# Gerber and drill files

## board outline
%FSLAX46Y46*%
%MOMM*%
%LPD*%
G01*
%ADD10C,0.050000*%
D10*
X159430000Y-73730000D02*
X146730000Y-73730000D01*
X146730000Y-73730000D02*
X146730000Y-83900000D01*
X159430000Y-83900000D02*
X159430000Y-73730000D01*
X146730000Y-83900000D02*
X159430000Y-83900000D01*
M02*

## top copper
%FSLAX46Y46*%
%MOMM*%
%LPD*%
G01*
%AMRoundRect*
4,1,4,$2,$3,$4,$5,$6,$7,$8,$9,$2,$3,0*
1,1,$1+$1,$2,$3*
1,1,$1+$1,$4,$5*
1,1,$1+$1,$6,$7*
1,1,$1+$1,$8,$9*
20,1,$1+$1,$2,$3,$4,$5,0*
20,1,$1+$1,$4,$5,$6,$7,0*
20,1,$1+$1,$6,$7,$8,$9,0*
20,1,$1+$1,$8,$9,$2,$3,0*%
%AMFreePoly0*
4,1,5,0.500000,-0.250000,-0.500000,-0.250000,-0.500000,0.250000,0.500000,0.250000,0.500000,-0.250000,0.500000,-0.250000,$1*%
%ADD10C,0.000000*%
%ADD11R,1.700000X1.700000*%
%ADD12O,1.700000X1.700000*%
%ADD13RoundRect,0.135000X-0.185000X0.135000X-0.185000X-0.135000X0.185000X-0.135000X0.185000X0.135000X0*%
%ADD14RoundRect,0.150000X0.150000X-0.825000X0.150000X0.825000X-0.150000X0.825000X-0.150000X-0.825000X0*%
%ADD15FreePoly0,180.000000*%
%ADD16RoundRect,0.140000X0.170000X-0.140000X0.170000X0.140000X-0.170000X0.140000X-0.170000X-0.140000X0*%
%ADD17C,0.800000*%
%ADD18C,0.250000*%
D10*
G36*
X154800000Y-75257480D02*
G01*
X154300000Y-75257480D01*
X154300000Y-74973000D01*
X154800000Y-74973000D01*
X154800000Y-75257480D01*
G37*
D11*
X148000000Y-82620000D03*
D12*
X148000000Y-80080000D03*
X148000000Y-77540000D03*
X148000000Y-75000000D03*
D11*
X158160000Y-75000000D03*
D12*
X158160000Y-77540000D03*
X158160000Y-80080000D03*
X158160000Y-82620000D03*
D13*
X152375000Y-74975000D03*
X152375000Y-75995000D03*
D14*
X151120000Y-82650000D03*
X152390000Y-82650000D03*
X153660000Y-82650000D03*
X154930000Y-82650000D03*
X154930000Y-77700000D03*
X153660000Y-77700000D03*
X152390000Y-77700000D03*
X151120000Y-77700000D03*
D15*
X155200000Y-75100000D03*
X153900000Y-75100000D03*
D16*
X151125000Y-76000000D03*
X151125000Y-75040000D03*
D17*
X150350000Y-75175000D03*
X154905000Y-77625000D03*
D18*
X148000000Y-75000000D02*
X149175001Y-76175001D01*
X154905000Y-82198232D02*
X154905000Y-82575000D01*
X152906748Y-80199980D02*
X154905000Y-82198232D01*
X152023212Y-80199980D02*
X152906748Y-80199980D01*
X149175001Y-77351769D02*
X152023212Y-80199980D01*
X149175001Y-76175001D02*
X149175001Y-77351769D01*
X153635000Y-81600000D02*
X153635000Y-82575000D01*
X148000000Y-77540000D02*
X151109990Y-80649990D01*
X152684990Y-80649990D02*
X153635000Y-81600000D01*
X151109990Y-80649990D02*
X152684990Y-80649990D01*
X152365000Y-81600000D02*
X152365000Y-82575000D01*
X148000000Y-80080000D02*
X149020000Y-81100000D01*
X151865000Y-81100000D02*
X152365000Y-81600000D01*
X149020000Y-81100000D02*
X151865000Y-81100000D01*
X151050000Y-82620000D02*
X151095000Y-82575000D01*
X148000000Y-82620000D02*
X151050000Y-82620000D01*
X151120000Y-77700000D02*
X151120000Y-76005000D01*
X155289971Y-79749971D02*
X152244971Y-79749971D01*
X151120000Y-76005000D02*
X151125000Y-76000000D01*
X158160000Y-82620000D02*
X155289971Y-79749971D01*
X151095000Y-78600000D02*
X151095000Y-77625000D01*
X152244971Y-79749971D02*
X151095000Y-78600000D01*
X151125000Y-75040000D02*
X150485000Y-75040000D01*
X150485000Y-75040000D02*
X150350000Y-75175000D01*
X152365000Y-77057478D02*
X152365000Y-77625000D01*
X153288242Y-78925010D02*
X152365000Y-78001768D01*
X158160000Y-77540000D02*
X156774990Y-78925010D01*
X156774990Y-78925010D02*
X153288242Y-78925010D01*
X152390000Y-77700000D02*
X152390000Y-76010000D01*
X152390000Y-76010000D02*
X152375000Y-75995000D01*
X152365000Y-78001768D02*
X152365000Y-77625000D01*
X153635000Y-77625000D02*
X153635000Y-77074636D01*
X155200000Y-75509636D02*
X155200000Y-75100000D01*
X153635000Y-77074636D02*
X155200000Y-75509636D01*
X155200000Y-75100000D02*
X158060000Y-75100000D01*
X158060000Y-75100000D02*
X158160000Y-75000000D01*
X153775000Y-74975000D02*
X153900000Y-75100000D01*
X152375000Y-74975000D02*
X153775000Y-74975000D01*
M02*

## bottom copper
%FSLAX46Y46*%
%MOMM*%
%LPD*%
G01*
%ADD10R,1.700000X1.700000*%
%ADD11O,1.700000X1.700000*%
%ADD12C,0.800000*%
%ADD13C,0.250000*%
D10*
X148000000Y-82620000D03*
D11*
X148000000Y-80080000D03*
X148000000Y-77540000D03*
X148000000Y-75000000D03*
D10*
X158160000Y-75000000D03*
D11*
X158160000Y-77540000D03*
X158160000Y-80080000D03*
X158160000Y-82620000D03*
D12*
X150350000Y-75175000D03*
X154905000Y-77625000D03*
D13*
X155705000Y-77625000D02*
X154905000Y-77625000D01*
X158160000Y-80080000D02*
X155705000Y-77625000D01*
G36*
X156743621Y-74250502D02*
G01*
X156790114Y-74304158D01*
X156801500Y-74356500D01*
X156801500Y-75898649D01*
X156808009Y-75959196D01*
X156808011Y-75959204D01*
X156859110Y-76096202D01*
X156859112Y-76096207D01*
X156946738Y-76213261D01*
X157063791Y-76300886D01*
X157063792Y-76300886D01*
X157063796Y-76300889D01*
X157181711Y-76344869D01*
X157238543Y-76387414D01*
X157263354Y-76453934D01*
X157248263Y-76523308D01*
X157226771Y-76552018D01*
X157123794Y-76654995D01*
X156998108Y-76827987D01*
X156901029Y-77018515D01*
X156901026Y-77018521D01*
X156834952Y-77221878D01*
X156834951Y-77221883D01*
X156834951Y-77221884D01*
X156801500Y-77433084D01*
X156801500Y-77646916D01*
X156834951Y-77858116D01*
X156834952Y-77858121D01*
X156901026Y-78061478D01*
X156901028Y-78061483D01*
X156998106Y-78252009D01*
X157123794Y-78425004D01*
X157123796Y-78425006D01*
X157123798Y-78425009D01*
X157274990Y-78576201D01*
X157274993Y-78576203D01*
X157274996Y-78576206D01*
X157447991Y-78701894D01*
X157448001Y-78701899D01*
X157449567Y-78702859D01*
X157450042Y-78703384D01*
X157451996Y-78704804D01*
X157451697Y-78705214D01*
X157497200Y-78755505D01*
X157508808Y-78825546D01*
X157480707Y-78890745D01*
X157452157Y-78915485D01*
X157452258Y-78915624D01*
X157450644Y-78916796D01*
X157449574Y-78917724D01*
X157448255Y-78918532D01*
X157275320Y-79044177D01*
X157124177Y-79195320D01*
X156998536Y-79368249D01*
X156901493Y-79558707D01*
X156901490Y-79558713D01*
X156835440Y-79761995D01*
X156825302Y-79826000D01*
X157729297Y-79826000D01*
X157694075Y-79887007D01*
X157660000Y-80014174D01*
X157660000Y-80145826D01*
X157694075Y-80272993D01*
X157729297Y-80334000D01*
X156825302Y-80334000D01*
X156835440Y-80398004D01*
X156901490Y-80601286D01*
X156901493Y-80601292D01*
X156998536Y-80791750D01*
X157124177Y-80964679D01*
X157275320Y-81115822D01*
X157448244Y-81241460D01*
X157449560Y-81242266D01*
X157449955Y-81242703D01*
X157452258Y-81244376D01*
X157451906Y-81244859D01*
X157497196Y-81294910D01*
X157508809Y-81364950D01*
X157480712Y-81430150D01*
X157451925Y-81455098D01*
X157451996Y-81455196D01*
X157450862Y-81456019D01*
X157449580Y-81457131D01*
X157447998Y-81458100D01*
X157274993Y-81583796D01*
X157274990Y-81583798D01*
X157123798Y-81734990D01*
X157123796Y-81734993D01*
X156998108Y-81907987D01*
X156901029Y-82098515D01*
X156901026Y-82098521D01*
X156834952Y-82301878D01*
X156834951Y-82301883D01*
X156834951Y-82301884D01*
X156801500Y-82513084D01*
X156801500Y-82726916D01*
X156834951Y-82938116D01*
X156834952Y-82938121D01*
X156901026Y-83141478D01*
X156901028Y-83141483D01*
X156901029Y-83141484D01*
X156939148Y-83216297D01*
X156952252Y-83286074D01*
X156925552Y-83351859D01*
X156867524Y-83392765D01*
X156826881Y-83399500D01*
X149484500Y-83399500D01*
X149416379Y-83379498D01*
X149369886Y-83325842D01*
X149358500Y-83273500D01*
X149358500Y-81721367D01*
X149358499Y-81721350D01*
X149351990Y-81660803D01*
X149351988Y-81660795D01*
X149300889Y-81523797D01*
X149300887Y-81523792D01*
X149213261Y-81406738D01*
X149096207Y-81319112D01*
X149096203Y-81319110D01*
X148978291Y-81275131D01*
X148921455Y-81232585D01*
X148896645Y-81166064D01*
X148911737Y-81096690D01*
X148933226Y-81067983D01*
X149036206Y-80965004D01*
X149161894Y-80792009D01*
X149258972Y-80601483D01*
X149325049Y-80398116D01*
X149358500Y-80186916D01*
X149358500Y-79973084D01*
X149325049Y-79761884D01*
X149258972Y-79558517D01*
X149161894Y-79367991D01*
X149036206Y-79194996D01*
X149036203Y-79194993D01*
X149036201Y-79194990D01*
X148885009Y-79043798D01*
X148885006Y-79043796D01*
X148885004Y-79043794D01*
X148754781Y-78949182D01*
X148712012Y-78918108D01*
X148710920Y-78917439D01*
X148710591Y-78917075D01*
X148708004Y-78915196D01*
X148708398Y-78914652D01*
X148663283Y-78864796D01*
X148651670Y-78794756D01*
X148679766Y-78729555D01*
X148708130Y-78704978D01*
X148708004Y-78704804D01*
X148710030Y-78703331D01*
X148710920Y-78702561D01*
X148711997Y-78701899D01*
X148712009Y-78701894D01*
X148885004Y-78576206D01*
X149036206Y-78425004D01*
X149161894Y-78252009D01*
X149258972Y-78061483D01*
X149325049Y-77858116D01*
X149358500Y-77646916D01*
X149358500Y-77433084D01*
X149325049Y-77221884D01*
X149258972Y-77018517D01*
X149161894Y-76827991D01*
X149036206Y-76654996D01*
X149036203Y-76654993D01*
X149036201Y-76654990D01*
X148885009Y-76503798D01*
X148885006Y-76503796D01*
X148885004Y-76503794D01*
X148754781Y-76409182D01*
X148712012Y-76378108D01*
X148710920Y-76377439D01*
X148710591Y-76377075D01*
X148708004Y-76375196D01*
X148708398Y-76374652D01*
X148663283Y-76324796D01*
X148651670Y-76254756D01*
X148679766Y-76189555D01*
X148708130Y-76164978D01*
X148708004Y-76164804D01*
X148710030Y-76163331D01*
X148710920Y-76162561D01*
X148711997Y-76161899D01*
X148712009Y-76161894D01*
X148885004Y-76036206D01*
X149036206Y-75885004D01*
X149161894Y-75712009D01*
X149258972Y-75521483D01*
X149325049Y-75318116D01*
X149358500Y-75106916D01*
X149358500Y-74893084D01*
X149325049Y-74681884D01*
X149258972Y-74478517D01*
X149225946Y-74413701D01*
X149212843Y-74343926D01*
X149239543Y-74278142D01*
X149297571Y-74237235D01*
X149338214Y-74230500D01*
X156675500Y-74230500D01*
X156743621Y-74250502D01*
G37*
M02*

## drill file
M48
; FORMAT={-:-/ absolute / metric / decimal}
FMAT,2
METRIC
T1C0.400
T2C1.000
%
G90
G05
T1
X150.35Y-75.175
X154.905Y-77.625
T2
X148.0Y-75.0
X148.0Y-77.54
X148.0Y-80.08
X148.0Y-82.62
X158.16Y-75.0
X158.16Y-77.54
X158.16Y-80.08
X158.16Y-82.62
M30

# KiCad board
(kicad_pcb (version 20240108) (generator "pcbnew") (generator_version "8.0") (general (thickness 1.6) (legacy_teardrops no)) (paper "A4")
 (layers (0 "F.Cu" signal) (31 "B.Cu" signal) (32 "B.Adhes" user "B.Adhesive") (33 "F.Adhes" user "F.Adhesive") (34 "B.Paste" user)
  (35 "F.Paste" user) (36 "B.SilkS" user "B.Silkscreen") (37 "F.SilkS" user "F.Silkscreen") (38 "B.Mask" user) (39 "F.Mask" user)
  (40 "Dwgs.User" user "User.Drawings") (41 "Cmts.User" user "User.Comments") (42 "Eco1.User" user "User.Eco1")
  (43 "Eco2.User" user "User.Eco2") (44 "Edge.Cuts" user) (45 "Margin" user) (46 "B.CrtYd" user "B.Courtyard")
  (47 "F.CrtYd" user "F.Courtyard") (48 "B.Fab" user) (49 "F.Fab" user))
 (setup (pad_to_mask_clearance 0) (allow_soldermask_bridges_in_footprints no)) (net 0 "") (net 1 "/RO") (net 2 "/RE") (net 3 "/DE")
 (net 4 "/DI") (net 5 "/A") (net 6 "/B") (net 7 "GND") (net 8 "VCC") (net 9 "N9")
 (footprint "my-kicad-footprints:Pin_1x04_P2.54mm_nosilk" (layer "F.Cu") (at 148 82.62 180)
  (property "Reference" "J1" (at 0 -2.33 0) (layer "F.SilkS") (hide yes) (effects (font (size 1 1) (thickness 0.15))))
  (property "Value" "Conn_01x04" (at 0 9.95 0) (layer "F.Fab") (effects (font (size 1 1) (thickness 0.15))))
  (pad "1" thru_hole rect (at 0 0 180) (size 1.7 1.7) (drill 1) (layers "*.Cu" "*.Mask") (remove_unused_layers no) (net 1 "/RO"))
  (pad "2" thru_hole oval (at 0 2.54 180) (size 1.7 1.7) (drill 1) (layers "*.Cu" "*.Mask") (remove_unused_layers no) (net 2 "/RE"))
  (pad "3" thru_hole oval (at 0 5.08 180) (size 1.7 1.7) (drill 1) (layers "*.Cu" "*.Mask") (remove_unused_layers no) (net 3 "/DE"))
  (pad "4" thru_hole oval (at 0 7.62 180) (size 1.7 1.7) (drill 1) (layers "*.Cu" "*.Mask") (remove_unused_layers no) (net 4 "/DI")))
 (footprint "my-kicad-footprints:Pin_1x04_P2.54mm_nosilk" (layer "F.Cu") (at 158.16 75)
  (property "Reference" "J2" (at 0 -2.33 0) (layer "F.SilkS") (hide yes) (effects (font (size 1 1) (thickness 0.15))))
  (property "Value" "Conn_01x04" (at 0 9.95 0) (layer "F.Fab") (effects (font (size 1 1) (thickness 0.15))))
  (pad "1" thru_hole rect (at 0 0) (size 1.7 1.7) (drill 1) (layers "*.Cu" "*.Mask") (remove_unused_layers no) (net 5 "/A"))
  (pad "2" thru_hole oval (at 0 2.54) (size 1.7 1.7) (drill 1) (layers "*.Cu" "*.Mask") (remove_unused_layers no) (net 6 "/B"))
  (pad "3" thru_hole oval (at 0 5.08) (size 1.7 1.7) (drill 1) (layers "*.Cu" "*.Mask") (remove_unused_layers no) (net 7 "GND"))
  (pad "4" thru_hole oval (at 0 7.62) (size 1.7 1.7) (drill 1) (layers "*.Cu" "*.Mask") (remove_unused_layers no) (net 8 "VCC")))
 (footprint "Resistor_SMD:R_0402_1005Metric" (layer "F.Cu") (at 152.375 75.485 -90)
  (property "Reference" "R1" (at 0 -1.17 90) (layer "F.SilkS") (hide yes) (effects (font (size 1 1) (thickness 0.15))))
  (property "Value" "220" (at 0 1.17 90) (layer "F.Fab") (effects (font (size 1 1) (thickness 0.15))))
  (pad "1" smd roundrect (at -0.51 0 270) (size 0.54 0.64) (layers "F.Cu" "F.Paste" "F.Mask") (roundrect_rratio 0.25) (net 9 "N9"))
  (pad "2" smd roundrect (at 0.51 0 270) (size 0.54 0.64) (layers "F.Cu" "F.Paste" "F.Mask") (roundrect_rratio 0.25) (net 6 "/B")))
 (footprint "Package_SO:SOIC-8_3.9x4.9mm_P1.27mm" (layer "F.Cu") (at 153.025 80.175 90)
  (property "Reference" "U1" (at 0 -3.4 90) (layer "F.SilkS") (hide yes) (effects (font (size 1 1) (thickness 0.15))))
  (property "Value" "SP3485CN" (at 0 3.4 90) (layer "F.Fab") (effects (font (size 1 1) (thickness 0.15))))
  (pad "1" smd roundrect (at -2.475 -1.905 90) (size 1.95 0.6) (layers "F.Cu" "F.Paste" "F.Mask") (roundrect_rratio 0.25) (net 1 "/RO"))
  (pad "2" smd roundrect (at -2.475 -0.635 90) (size 1.95 0.6) (layers "F.Cu" "F.Paste" "F.Mask") (roundrect_rratio 0.25) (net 2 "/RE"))
  (pad "3" smd roundrect (at -2.475 0.635 90) (size 1.95 0.6) (layers "F.Cu" "F.Paste" "F.Mask") (roundrect_rratio 0.25) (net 3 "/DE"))
  (pad "4" smd roundrect (at -2.475 1.905 90) (size 1.95 0.6) (layers "F.Cu" "F.Paste" "F.Mask") (roundrect_rratio 0.25) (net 4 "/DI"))
  (pad "5" smd roundrect (at 2.475 1.905 90) (size 1.95 0.6) (layers "F.Cu" "F.Paste" "F.Mask") (roundrect_rratio 0.25) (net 7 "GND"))
  (pad "6" smd roundrect (at 2.475 0.635 90) (size 1.95 0.6) (layers "F.Cu" "F.Paste" "F.Mask") (roundrect_rratio 0.25) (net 5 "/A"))
  (pad "7" smd roundrect (at 2.475 -0.635 90) (size 1.95 0.6) (layers "F.Cu" "F.Paste" "F.Mask") (roundrect_rratio 0.25) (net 6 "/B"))
  (pad "8" smd roundrect (at 2.475 -1.905 90) (size 1.95 0.6) (layers "F.Cu" "F.Paste" "F.Mask") (roundrect_rratio 0.25) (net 8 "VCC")))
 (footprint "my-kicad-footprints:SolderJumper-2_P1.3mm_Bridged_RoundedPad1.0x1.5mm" (layer "F.Cu") (at 154.55 75.1 180)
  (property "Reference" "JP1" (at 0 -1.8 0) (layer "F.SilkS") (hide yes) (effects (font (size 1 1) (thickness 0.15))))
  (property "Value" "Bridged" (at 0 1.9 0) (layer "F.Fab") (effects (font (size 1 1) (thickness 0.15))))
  (fp_poly
   (pts (xy 0.25 -0.15748) (xy -0.25 -0.15748) (xy -0.25 0.127) (xy 0.25 0.127)) (stroke (width 0) (type solid)) (fill solid) (layer "F.Cu"))
  (pad "1" smd custom (at -0.65 0 180) (size 1 0.5) (layers "F.Cu" "F.Mask") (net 5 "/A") (zone_connect 2)
   (options (clearance outline) (anchor rect)) (primitives))
  (pad "2" smd custom (at 0.65 0 180) (size 1 0.5) (layers "F.Cu" "F.Mask") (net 9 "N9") (zone_connect 2)
   (options (clearance outline) (anchor rect)) (primitives)))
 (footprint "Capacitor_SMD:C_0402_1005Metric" (layer "F.Cu") (at 151.125 75.52 90)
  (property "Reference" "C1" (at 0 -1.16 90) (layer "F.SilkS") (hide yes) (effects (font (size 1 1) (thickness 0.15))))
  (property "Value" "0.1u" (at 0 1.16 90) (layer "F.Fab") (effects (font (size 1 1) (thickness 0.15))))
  (pad "1" smd roundrect (at -0.48 0 90) (size 0.56 0.62) (layers "F.Cu" "F.Paste" "F.Mask") (roundrect_rratio 0.25) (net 8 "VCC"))
  (pad "2" smd roundrect (at 0.48 0 90) (size 0.56 0.62) (layers "F.Cu" "F.Paste" "F.Mask") (roundrect_rratio 0.25) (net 7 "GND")))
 (gr_line (start 159.43 73.73) (end 146.73 73.73) (stroke (width 0.05) (type solid)) (layer "Edge.Cuts"))
 (gr_line (start 146.73 73.73) (end 146.73 83.9) (stroke (width 0.05) (type solid)) (layer "Edge.Cuts"))
 (gr_line (start 159.43 83.9) (end 159.43 73.73) (stroke (width 0.05) (type solid)) (layer "Edge.Cuts"))
 (gr_line (start 146.73 83.9) (end 159.43 83.9) (stroke (width 0.05) (type solid)) (layer "Edge.Cuts"))
 (segment (start 148 75) (end 149.175001 76.175001) (width 0.25) (layer "F.Cu") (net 4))
 (segment (start 154.905 82.198232) (end 154.905 82.575) (width 0.25) (layer "F.Cu") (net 4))
 (segment (start 152.906748 80.19998) (end 154.905 82.198232) (width 0.25) (layer "F.Cu") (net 4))
 (segment (start 152.023212 80.19998) (end 152.906748 80.19998) (width 0.25) (layer "F.Cu") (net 4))
 (segment (start 149.175001 77.351769) (end 152.023212 80.19998) (width 0.25) (layer "F.Cu") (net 4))
 (segment (start 149.175001 76.175001) (end 149.175001 77.351769) (width 0.25) (layer "F.Cu") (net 4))
 (segment (start 153.635 81.6) (end 153.635 82.575) (width 0.25) (layer "F.Cu") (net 3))
 (segment (start 148 77.54) (end 151.10999 80.64999) (width 0.25) (layer "F.Cu") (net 3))
 (segment (start 152.68499 80.64999) (end 153.635 81.6) (width 0.25) (layer "F.Cu") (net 3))
 (segment (start 151.10999 80.64999) (end 152.68499 80.64999) (width 0.25) (layer "F.Cu") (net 3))
 (segment (start 152.365 81.6) (end 152.365 82.575) (width 0.25) (layer "F.Cu") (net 2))
 (segment (start 148 80.08) (end 149.02 81.1) (width 0.25) (layer "F.Cu") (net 2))
 (segment (start 151.865 81.1) (end 152.365 81.6) (width 0.25) (layer "F.Cu") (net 2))
 (segment (start 149.02 81.1) (end 151.865 81.1) (width 0.25) (layer "F.Cu") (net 2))
 (segment (start 151.05 82.62) (end 151.095 82.575) (width 0.25) (layer "F.Cu") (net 1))
 (segment (start 148 82.62) (end 151.05 82.62) (width 0.25) (layer "F.Cu") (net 1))
 (segment (start 151.12 77.7) (end 151.12 76.005) (width 0.25) (layer "F.Cu") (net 8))
 (segment (start 155.289971 79.749971) (end 152.244971 79.749971) (width 0.25) (layer "F.Cu") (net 8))
 (segment (start 151.12 76.005) (end 151.125 76) (width 0.25) (layer "F.Cu") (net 8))
 (segment (start 158.16 82.62) (end 155.289971 79.749971) (width 0.25) (layer "F.Cu") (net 8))
 (segment (start 151.095 78.6) (end 151.095 77.625) (width 0.25) (layer "F.Cu") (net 8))
 (segment (start 152.244971 79.749971) (end 151.095 78.6) (width 0.25) (layer "F.Cu") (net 8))
 (segment (start 151.125 75.04) (end 150.485 75.04) (width 0.25) (layer "F.Cu") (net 7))
 (segment (start 150.485 75.04) (end 150.35 75.175) (width 0.25) (layer "F.Cu") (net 7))
 (via (at 150.35 75.175) (size 0.8) (drill 0.4) (layers "F.Cu" "B.Cu") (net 7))
 (via (at 154.905 77.625) (size 0.8) (drill 0.4) (layers "F.Cu" "B.Cu") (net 7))
 (segment (start 155.705 77.625) (end 154.905 77.625) (width 0.25) (layer "B.Cu") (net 7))
 (segment (start 158.16 80.08) (end 155.705 77.625) (width 0.25) (layer "B.Cu") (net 7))
 (segment (start 152.365 77.057478) (end 152.365 77.625) (width 0.25) (layer "F.Cu") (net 6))
 (segment (start 153.288242 78.92501) (end 152.365 78.001768) (width 0.25) (layer "F.Cu") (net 6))
 (segment (start 158.16 77.54) (end 156.77499 78.92501) (width 0.25) (layer "F.Cu") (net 6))
 (segment (start 156.77499 78.92501) (end 153.288242 78.92501) (width 0.25) (layer "F.Cu") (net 6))
 (segment (start 152.39 77.7) (end 152.39 76.01) (width 0.25) (layer "F.Cu") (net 6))
 (segment (start 152.39 76.01) (end 152.375 75.995) (width 0.25) (layer "F.Cu") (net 6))
 (segment (start 152.365 78.001768) (end 152.365 77.625) (width 0.25) (layer "F.Cu") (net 6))
 (segment (start 153.635 77.625) (end 153.635 77.074636) (width 0.25) (layer "F.Cu") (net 5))
 (segment (start 155.2 75.509636) (end 155.2 75.1) (width 0.25) (layer "F.Cu") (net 5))
 (segment (start 153.635 77.074636) (end 155.2 75.509636) (width 0.25) (layer "F.Cu") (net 5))
 (segment (start 155.2 75.1) (end 158.06 75.1) (width 0.25) (layer "F.Cu") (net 5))
 (segment (start 158.06 75.1) (end 158.16 75) (width 0.25) (layer "F.Cu") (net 5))
 (segment (start 153.775 74.975) (end 153.9 75.1) (width 0.25) (layer "F.Cu") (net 9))
 (segment (start 152.375 74.975) (end 153.775 74.975) (width 0.25) (layer "F.Cu") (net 9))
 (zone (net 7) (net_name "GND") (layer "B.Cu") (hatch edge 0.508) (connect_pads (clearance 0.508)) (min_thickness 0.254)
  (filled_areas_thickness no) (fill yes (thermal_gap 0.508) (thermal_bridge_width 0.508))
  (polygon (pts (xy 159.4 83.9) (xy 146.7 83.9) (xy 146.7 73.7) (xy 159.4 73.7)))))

